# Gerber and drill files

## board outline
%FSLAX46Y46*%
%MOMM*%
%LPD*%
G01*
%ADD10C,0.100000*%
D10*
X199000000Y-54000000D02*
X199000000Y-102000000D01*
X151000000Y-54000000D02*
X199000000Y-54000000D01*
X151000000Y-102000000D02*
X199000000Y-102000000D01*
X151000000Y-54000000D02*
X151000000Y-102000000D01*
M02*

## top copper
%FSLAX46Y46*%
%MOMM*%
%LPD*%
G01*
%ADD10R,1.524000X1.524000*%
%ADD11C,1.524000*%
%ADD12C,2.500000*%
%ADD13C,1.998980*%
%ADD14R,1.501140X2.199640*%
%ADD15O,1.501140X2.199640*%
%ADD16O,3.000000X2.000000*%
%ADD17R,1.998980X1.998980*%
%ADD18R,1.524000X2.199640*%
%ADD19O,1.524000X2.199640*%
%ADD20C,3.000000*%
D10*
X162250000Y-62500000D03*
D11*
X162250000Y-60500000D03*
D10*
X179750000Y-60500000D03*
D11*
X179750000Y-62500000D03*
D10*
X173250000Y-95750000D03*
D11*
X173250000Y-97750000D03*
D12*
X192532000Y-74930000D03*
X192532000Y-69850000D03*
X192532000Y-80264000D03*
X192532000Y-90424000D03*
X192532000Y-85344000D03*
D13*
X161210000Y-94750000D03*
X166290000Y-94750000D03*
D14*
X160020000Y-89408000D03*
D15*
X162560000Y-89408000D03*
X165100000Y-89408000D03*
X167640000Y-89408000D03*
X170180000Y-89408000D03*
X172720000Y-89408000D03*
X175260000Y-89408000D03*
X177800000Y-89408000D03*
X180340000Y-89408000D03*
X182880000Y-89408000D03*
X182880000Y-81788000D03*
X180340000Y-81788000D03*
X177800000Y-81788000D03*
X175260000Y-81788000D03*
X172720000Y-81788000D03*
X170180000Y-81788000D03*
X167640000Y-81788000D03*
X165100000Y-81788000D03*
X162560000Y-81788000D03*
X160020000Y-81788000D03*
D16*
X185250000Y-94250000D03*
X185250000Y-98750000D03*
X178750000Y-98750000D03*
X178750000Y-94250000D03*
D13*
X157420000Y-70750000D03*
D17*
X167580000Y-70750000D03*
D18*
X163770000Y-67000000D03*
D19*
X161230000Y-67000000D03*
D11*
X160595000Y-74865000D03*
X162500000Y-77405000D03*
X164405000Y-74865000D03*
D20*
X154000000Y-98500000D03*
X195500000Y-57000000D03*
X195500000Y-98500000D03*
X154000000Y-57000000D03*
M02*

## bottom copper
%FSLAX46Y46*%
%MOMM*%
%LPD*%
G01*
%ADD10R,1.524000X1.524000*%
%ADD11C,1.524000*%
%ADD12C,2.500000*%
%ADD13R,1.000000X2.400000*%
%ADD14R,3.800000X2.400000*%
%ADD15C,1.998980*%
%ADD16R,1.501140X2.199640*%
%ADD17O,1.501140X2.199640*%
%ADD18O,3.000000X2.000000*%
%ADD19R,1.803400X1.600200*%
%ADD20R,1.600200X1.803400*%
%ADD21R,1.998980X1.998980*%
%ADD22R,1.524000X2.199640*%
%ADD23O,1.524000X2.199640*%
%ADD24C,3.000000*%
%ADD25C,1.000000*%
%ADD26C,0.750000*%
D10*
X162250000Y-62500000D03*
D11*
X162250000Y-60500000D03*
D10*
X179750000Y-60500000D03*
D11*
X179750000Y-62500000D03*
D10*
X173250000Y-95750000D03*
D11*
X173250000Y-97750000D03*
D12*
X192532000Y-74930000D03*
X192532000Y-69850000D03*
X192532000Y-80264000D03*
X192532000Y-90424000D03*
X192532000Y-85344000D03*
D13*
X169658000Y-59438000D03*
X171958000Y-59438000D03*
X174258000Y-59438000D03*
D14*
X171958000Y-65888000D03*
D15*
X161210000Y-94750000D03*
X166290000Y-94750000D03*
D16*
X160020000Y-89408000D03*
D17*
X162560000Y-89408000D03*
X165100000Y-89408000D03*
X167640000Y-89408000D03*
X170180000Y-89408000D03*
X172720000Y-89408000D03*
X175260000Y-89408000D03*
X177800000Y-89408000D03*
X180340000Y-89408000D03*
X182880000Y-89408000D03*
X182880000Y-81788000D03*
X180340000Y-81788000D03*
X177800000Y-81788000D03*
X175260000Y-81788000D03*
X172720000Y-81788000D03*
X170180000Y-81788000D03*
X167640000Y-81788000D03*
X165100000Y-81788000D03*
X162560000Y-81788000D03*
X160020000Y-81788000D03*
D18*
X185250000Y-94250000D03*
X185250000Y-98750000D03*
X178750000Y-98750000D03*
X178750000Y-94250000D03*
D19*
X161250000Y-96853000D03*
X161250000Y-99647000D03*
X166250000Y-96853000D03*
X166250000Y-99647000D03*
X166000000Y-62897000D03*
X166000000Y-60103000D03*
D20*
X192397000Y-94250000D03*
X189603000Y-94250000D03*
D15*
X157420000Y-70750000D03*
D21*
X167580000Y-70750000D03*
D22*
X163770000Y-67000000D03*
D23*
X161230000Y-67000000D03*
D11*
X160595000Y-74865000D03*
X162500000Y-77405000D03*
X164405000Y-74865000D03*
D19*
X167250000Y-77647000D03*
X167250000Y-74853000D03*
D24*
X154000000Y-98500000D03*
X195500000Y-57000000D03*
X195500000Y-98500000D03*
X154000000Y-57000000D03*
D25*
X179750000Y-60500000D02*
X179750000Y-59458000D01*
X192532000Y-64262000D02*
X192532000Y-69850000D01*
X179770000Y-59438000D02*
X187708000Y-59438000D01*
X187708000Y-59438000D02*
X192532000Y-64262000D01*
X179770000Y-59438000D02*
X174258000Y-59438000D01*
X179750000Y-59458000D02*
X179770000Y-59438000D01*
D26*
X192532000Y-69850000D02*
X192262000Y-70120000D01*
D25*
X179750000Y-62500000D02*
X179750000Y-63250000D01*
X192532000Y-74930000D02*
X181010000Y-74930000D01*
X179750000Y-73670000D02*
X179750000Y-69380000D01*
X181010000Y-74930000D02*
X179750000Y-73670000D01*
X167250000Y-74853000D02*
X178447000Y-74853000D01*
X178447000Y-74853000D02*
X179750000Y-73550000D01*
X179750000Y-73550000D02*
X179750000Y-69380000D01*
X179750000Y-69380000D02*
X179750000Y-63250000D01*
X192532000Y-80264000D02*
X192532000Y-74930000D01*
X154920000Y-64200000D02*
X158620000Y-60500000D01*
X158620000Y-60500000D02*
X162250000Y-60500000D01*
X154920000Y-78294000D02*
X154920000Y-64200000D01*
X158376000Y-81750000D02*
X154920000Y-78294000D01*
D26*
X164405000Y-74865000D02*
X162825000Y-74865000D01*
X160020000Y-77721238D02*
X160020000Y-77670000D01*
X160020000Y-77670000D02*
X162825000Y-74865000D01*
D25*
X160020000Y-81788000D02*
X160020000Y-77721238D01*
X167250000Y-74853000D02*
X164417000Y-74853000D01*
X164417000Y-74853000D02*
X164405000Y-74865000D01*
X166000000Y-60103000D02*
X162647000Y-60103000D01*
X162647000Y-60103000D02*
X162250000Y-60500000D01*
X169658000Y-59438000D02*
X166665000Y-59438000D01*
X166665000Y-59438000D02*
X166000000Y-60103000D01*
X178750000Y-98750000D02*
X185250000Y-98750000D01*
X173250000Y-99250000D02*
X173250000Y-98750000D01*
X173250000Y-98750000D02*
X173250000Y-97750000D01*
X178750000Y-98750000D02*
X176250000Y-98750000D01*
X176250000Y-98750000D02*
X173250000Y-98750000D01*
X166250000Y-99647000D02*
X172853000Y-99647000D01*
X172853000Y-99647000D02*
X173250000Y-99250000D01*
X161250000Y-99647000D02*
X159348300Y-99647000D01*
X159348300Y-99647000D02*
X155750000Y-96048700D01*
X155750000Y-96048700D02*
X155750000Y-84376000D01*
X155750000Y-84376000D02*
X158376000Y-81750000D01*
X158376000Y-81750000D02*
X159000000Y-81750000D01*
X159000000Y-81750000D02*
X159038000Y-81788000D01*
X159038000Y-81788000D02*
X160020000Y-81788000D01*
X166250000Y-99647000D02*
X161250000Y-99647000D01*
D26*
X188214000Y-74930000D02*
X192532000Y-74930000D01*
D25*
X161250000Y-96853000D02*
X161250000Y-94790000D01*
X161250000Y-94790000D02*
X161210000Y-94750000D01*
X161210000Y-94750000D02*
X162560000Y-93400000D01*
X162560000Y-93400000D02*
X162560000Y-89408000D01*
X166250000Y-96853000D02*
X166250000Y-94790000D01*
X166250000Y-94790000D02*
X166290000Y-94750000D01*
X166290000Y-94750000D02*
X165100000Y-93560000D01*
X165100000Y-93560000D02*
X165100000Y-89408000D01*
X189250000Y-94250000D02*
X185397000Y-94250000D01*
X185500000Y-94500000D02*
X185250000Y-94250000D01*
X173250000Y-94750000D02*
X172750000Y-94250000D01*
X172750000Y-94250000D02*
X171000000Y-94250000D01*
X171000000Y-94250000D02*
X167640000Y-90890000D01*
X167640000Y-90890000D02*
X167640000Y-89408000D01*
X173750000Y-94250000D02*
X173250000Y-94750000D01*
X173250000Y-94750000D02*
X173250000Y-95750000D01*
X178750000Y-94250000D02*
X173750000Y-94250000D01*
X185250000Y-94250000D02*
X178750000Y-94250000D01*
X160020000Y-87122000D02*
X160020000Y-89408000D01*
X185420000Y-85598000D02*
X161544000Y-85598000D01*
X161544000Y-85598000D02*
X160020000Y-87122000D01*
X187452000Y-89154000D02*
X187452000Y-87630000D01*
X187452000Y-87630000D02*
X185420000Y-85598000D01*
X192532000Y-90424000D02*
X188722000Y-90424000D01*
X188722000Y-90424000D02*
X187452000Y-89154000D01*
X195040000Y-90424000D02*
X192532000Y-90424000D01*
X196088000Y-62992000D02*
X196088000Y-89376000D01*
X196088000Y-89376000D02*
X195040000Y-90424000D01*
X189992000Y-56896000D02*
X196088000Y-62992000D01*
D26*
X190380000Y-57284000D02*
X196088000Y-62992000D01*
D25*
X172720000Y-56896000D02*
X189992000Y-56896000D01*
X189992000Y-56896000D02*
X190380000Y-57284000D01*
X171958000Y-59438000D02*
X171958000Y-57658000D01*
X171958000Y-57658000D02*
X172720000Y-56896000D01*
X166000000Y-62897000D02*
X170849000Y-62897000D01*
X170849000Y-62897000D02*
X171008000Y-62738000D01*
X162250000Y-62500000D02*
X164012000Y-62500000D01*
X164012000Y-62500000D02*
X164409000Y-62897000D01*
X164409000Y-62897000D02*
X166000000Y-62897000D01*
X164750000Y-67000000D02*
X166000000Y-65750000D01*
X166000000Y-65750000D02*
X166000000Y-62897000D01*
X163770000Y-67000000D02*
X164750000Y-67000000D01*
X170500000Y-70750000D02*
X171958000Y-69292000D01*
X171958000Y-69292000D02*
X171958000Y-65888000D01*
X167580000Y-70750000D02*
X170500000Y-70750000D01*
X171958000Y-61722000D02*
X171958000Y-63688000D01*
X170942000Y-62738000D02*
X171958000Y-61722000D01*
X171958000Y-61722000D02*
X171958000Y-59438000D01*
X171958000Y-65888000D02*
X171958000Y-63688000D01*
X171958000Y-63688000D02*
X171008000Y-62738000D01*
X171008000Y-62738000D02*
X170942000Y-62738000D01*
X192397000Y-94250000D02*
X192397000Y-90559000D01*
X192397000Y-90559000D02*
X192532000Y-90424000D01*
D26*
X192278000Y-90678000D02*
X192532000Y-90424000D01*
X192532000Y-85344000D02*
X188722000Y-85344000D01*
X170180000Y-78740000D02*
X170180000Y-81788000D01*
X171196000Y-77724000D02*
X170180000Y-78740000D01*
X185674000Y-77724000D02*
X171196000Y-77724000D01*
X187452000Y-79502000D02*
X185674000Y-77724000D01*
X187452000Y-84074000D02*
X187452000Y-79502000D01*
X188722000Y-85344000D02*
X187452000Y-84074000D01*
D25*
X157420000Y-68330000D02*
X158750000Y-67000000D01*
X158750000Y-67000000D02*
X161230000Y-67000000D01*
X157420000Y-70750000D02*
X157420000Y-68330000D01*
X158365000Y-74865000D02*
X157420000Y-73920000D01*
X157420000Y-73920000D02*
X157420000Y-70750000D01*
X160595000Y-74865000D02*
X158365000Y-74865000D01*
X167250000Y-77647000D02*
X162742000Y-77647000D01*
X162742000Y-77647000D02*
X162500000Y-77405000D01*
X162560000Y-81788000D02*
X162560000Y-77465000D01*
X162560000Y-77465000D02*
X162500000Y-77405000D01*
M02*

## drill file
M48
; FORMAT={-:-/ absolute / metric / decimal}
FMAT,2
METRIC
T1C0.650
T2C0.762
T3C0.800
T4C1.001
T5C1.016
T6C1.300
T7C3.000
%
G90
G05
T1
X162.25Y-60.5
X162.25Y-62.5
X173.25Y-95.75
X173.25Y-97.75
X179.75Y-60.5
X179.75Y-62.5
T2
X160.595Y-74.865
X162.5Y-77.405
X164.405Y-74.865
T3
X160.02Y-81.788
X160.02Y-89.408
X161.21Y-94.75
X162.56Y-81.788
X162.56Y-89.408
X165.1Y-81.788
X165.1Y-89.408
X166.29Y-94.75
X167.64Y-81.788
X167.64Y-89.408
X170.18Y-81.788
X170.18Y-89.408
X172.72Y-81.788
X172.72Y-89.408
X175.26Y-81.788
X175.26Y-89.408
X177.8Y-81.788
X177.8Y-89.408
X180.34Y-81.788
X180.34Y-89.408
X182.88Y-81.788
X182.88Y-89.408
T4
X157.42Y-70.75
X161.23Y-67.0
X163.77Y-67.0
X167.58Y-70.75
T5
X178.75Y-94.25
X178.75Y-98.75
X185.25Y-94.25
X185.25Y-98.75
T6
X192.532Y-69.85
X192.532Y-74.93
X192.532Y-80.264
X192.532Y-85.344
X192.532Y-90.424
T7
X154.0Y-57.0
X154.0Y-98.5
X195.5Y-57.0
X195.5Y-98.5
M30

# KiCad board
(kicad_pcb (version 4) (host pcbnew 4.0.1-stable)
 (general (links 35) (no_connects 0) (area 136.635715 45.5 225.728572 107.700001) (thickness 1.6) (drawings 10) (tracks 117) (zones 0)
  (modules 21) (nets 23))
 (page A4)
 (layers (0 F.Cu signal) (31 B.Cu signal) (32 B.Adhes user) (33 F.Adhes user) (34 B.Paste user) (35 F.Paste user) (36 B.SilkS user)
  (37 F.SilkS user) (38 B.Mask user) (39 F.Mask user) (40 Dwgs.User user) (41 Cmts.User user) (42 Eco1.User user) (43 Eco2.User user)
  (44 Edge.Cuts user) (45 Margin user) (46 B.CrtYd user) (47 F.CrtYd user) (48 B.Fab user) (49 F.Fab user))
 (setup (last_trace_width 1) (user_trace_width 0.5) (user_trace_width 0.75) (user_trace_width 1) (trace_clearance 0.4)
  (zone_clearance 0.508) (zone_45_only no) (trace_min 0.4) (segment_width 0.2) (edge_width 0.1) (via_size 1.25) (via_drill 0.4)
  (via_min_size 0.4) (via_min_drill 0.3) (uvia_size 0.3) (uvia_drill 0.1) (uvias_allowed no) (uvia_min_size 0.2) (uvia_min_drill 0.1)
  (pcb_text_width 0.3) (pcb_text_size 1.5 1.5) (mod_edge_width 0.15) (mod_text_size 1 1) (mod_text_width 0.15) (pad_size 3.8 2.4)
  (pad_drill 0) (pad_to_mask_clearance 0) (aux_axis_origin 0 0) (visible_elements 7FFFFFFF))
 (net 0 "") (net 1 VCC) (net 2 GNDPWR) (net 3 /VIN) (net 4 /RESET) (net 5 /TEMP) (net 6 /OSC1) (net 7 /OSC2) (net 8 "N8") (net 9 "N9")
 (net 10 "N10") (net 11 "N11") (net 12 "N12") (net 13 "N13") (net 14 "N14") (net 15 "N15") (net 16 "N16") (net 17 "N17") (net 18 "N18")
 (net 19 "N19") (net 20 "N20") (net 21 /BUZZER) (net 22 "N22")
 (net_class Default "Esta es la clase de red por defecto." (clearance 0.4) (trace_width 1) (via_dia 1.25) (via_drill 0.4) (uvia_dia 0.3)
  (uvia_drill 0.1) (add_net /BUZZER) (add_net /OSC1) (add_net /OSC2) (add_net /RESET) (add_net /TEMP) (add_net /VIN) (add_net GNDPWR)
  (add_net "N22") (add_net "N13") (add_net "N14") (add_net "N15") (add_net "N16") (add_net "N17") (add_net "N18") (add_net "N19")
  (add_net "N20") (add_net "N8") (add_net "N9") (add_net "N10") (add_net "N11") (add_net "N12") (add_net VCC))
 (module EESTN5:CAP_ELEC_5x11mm (layer F.Cu) (at 162.25 61.5)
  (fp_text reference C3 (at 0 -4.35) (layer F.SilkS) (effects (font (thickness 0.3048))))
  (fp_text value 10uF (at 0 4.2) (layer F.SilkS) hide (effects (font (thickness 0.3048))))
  (pad 1 thru_hole rect (at 0 1) (size 1.524 1.524) (drill 0.65) (layers *.Cu *.Mask F.SilkS) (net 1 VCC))
  (pad 2 thru_hole circle (at 0 -1) (size 1.524 1.524) (drill 0.65) (layers *.Cu *.Mask F.SilkS) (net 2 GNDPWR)))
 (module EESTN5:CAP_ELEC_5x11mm (layer F.Cu) (at 179.75 61.5 180)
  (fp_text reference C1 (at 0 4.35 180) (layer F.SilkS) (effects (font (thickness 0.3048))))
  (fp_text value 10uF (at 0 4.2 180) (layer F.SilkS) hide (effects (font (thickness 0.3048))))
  (pad 1 thru_hole rect (at 0 1 180) (size 1.524 1.524) (drill 0.65) (layers *.Cu *.Mask F.SilkS) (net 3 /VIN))
  (pad 2 thru_hole circle (at 0 -1 180) (size 1.524 1.524) (drill 0.65) (layers *.Cu *.Mask F.SilkS) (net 2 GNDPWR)))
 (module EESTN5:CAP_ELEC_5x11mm (layer F.Cu) (at 173.25 96.75 180)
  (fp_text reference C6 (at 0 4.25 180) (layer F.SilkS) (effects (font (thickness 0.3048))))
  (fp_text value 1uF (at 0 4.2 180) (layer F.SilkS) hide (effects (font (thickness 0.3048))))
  (pad 1 thru_hole rect (at 0 1 180) (size 1.524 1.524) (drill 0.65) (layers *.Cu *.Mask F.SilkS) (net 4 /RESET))
  (pad 2 thru_hole circle (at 0 -1 180) (size 1.524 1.524) (drill 0.65) (layers *.Cu *.Mask F.SilkS) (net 2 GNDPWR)))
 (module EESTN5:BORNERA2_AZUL (layer F.Cu) (at 192.532 72.39 90)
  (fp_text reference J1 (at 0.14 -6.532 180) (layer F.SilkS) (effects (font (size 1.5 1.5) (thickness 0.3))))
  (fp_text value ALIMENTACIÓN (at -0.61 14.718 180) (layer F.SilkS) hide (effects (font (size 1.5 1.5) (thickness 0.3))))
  (pad 1 thru_hole circle (at -2.54 0 90) (size 2.5 2.5) (drill 1.3) (layers *.Cu *.Mask F.SilkS) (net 2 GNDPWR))
  (pad 2 thru_hole circle (at 2.54 0 90) (size 2.5 2.5) (drill 1.3) (layers *.Cu *.Mask F.SilkS) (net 3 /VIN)))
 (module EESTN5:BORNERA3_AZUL (layer F.Cu) (at 192.532 85.344 90)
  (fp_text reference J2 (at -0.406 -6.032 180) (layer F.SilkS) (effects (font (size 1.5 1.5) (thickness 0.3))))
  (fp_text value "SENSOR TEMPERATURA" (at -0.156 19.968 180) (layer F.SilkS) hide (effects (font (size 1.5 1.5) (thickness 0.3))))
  (pad 3 thru_hole circle (at 5.08 0 90) (size 2.5 2.5) (drill 1.3) (layers *.Cu *.Mask F.SilkS) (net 2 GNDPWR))
  (pad 1 thru_hole circle (at -5.08 0 90) (size 2.5 2.5) (drill 1.3) (layers *.Cu *.Mask F.SilkS) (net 1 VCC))
  (pad 2 thru_hole circle (at 0 0 90) (size 2.5 2.5) (drill 1.3) (layers *.Cu *.Mask F.SilkS) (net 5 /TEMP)))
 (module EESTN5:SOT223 (layer B.Cu) (at 171.958 62.738)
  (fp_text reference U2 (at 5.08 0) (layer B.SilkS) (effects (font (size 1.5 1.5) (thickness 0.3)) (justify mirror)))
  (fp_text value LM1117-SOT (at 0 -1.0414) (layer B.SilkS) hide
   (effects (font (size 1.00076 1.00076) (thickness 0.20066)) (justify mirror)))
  (pad 1 smd rect (at -2.3 -3.3) (size 1 2.4) (layers B.Cu B.Paste B.Mask) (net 2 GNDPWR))
  (pad 2 smd rect (at 0 -3.3) (size 1 2.4) (layers B.Cu B.Paste B.Mask) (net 1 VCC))
  (pad 3 smd rect (at 2.3 -3.3) (size 1 2.4) (layers B.Cu B.Paste B.Mask) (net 3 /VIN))
  (pad 4 smd rect (at 0 3.15) (size 3.8 2.4) (layers B.Cu B.Paste B.Mask)))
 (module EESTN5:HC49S (layer F.Cu) (at 163.75 94.75) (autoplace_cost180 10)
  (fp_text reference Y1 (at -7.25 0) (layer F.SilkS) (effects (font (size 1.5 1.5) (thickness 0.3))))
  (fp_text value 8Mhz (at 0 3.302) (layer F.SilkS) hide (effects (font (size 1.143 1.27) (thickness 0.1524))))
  (pad 1 thru_hole circle (at -2.54 0) (size 1.99898 1.99898) (drill 0.8001) (layers *.Cu *.Mask F.SilkS) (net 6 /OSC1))
  (pad 2 thru_hole circle (at 2.54 0) (size 1.99898 1.99898) (drill 0.8001) (layers *.Cu *.Mask F.SilkS) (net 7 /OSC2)))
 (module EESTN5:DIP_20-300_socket (layer F.Cu) (at 171.45 85.598)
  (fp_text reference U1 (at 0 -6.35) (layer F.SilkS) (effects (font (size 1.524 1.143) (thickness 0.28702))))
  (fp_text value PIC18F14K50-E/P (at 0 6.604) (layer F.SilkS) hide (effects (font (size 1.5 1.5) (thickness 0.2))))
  (pad 1 thru_hole rect (at -11.43 3.81) (size 1.50114 2.19964) (drill 0.8001) (layers *.Cu *.Mask F.SilkS) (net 1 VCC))
  (pad 2 thru_hole oval (at -8.89 3.81) (size 1.50114 2.19964) (drill 0.8001) (layers *.Cu *.Mask F.SilkS) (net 6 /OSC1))
  (pad 3 thru_hole oval (at -6.35 3.81) (size 1.50114 2.19964) (drill 0.8001) (layers *.Cu *.Mask F.SilkS) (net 7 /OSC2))
  (pad 4 thru_hole oval (at -3.81 3.81) (size 1.50114 2.19964) (drill 0.8001) (layers *.Cu *.Mask F.SilkS) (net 4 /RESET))
  (pad 5 thru_hole oval (at -1.27 3.81) (size 1.50114 2.19964) (drill 0.8001) (layers *.Cu *.Mask F.SilkS) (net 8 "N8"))
  (pad 6 thru_hole oval (at 1.27 3.81) (size 1.50114 2.19964) (drill 0.8001) (layers *.Cu *.Mask F.SilkS) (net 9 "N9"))
  (pad 7 thru_hole oval (at 3.81 3.81) (size 1.50114 2.19964) (drill 0.8001) (layers *.Cu *.Mask F.SilkS) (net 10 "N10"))
  (pad 8 thru_hole oval (at 6.35 3.81) (size 1.50114 2.19964) (drill 0.8001) (layers *.Cu *.Mask F.SilkS) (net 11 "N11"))
  (pad 9 thru_hole oval (at 8.89 3.81) (size 1.50114 2.19964) (drill 0.8001) (layers *.Cu *.Mask F.SilkS) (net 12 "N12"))
  (pad 10 thru_hole oval (at 11.43 3.81) (size 1.50114 2.19964) (drill 0.8001) (layers *.Cu *.Mask F.SilkS) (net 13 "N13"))
  (pad 11 thru_hole oval (at 11.43 -3.81) (size 1.50114 2.19964) (drill 0.8001) (layers *.Cu *.Mask F.SilkS) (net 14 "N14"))
  (pad 12 thru_hole oval (at 8.89 -3.81) (size 1.50114 2.19964) (drill 0.8001) (layers *.Cu *.Mask F.SilkS) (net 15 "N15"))
  (pad 13 thru_hole oval (at 6.35 -3.81) (size 1.50114 2.19964) (drill 0.8001) (layers *.Cu *.Mask F.SilkS) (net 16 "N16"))
  (pad 14 thru_hole oval (at 3.81 -3.81) (size 1.50114 2.19964) (drill 0.8001) (layers *.Cu *.Mask F.SilkS) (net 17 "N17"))
  (pad 15 thru_hole oval (at 1.27 -3.81) (size 1.50114 2.19964) (drill 0.8001) (layers *.Cu *.Mask F.SilkS) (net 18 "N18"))
  (pad 16 thru_hole oval (at -1.27 -3.81) (size 1.50114 2.19964) (drill 0.8001) (layers *.Cu *.Mask F.SilkS) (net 5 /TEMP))
  (pad 17 thru_hole oval (at -3.81 -3.81) (size 1.50114 2.19964) (drill 0.8001) (layers *.Cu *.Mask F.SilkS) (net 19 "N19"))
  (pad 18 thru_hole oval (at -6.35 -3.81) (size 1.50114 2.19964) (drill 0.8001) (layers *.Cu *.Mask F.SilkS) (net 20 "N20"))
  (pad 19 thru_hole oval (at -8.89 -3.81) (size 1.50114 2.19964) (drill 0.8001) (layers *.Cu *.Mask F.SilkS) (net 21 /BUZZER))
  (pad 20 thru_hole oval (at -11.43 -3.81) (size 1.50114 2.19964) (drill 0.8001) (layers *.Cu *.Mask F.SilkS) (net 2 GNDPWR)))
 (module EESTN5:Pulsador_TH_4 (layer F.Cu) (at 185.25 94.25 270)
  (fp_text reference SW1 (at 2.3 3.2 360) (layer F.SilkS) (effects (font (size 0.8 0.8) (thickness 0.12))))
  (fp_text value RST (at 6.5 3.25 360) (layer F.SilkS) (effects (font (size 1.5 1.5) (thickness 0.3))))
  (pad 3 thru_hole oval (at 0 0 270) (size 2 3) (drill 1.016) (layers *.Cu *.Mask F.SilkS) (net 4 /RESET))
  (pad 1 thru_hole oval (at 4.5 0 270) (size 2 3) (drill 1.016) (layers *.Cu *.Mask F.SilkS) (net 2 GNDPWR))
  (pad 2 thru_hole oval (at 4.5 6.5 270) (size 2 3) (drill 1.016) (layers *.Cu *.Mask F.SilkS) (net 2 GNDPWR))
  (pad 4 thru_hole oval (at 0 6.5 270) (size 2 3) (drill 1.016) (layers *.Cu *.Mask F.SilkS) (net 4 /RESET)))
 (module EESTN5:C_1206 (layer B.Cu) (at 161.25 98.25 90)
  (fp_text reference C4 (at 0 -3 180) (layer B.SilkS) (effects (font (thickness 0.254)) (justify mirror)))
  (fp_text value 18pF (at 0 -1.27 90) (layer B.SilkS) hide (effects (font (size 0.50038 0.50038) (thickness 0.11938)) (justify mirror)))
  (pad 1 smd rect (at 1.397 0 90) (size 1.6002 1.8034) (layers B.Cu B.Paste B.Mask) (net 6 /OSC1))
  (pad 2 smd rect (at -1.397 0 90) (size 1.6002 1.8034) (layers B.Cu B.Paste B.Mask) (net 2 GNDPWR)))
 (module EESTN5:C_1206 (layer B.Cu) (at 166.25 98.25 90)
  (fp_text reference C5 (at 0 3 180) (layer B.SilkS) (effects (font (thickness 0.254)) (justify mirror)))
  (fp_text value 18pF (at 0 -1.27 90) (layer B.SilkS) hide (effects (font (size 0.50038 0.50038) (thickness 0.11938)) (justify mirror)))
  (pad 1 smd rect (at 1.397 0 90) (size 1.6002 1.8034) (layers B.Cu B.Paste B.Mask) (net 7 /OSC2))
  (pad 2 smd rect (at -1.397 0 90) (size 1.6002 1.8034) (layers B.Cu B.Paste B.Mask) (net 2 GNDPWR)))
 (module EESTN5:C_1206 (layer B.Cu) (at 166 61.5 270)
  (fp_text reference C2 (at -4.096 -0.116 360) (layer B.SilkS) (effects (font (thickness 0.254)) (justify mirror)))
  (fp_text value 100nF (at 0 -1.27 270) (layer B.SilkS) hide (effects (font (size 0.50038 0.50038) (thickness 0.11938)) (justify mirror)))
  (pad 1 smd rect (at 1.397 0 270) (size 1.6002 1.8034) (layers B.Cu B.Paste B.Mask) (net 1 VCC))
  (pad 2 smd rect (at -1.397 0 270) (size 1.6002 1.8034) (layers B.Cu B.Paste B.Mask) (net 2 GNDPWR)))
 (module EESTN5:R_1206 (layer B.Cu) (at 191 94.25)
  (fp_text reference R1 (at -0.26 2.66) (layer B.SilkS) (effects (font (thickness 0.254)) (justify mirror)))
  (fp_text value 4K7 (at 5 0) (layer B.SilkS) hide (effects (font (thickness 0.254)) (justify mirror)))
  (pad 1 smd rect (at 1.397 0) (size 1.6002 1.8034) (layers B.Cu B.Paste B.Mask) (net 1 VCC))
  (pad 2 smd rect (at -1.397 0) (size 1.6002 1.8034) (layers B.Cu B.Paste B.Mask) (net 4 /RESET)))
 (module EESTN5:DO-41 (layer F.Cu) (at 162.5 70.75)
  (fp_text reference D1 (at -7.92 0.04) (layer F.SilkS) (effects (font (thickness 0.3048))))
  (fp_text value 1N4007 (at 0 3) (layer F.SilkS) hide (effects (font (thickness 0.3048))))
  (pad 1 thru_hole circle (at -5.08 0) (size 1.99898 1.99898) (drill 1.00076) (layers *.Cu *.Mask F.SilkS) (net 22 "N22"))
  (pad 2 thru_hole rect (at 5.08 0) (size 1.99898 1.99898) (drill 1.00076) (layers *.Cu *.Mask F.SilkS) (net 1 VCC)))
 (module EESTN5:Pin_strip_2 (layer F.Cu) (at 162.5 67 180)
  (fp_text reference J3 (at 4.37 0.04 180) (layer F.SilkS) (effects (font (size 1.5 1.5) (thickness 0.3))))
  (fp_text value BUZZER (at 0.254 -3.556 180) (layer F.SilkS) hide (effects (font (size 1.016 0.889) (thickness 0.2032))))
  (pad 1 thru_hole rect (at -1.27 0 180) (size 1.524 2.19964) (drill 1.00076) (layers *.Cu *.Mask F.SilkS) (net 1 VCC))
  (pad 2 thru_hole oval (at 1.27 0 180) (size 1.524 2.19964) (drill 1.00076) (layers *.Cu *.Mask F.SilkS) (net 22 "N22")))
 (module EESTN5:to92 (layer F.Cu) (at 162.5 75.5 180)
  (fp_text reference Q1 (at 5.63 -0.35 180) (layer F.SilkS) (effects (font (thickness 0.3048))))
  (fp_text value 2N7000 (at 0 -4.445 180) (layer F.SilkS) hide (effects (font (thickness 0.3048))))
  (pad 3 thru_hole circle (at 1.905 0.635 180) (size 1.524 1.524) (drill 0.762) (layers *.Cu *.Mask F.SilkS) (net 22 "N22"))
  (pad 2 thru_hole circle (at 0 -1.905 180) (size 1.524 1.524) (drill 0.762) (layers *.Cu *.Mask F.SilkS) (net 21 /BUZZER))
  (pad 1 thru_hole circle (at -1.905 0.635 180) (size 1.524 1.524) (drill 0.762) (layers *.Cu *.Mask F.SilkS) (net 2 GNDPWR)))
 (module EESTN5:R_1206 (layer B.Cu) (at 167.25 76.25 270)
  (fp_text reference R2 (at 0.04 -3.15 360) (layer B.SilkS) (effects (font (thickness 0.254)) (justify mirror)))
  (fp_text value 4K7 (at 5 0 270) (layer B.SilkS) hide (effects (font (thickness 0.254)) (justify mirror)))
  (pad 1 smd rect (at 1.397 0 270) (size 1.6002 1.8034) (layers B.Cu B.Paste B.Mask) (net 21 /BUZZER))
  (pad 2 smd rect (at -1.397 0 270) (size 1.6002 1.8034) (layers B.Cu B.Paste B.Mask) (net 2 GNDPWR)))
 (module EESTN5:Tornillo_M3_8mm (layer F.Cu) (at 154 98.5)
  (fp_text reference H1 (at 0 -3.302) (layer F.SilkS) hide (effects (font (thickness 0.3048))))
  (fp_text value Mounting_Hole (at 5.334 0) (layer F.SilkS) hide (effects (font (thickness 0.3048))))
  (pad 1 thru_hole circle (at 0 0) (size 3 3) (drill 3) (layers *.Cu F.SilkS)))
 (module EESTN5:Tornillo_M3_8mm (layer F.Cu) (at 195.5 57)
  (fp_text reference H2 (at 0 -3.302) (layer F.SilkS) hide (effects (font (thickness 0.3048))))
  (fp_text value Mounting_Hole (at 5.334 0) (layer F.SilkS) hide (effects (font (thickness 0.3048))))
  (pad 1 thru_hole circle (at 0 0) (size 3 3) (drill 3) (layers *.Cu F.SilkS)))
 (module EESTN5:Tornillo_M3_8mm (layer F.Cu) (at 195.5 98.5)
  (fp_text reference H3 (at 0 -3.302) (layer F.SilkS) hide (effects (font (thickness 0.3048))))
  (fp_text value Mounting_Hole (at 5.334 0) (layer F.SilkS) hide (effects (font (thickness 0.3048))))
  (pad 1 thru_hole circle (at 0 0) (size 3 3) (drill 3) (layers *.Cu F.SilkS)))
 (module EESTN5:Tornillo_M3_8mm (layer F.Cu) (at 154 57)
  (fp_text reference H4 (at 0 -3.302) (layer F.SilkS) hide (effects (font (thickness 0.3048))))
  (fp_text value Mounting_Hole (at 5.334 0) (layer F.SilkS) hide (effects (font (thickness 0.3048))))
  (pad 1 thru_hole circle (at 0 0) (size 3 3) (drill 3) (layers *.Cu F.SilkS)))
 (gr_line (start 199 54) (end 199 102) (angle 90) (layer Edge.Cuts) (width 0.1))
 (gr_line (start 151 54) (end 199 54) (angle 90) (layer Edge.Cuts) (width 0.1))
 (gr_line (start 151 102) (end 199 102) (angle 90) (layer Edge.Cuts) (width 0.1))
 (gr_line (start 151 54) (end 151 102) (angle 90) (layer Edge.Cuts) (width 0.1))
 (segment (start 179.75 60.5) (end 179.75 59.458) (width 1) (layer B.Cu) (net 3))
 (segment (start 192.532 64.262) (end 192.532 69.85) (width 1) (layer B.Cu) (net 3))
 (segment (start 179.77 59.438) (end 187.708 59.438) (width 1) (layer B.Cu) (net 3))
 (segment (start 187.708 59.438) (end 192.532 64.262) (width 1) (layer B.Cu) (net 3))
 (segment (start 179.77 59.438) (end 174.258 59.438) (width 1) (layer B.Cu) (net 3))
 (segment (start 179.75 59.458) (end 179.77 59.438) (width 1) (layer B.Cu) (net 3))
 (segment (start 192.532 69.85) (end 192.262 70.12) (width 0.75) (layer B.Cu) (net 3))
 (segment (start 179.75 62.5) (end 179.75 63.25) (width 1) (layer B.Cu) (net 2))
 (segment (start 192.532 74.93) (end 181.01 74.93) (width 1) (layer B.Cu) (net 2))
 (segment (start 179.75 73.67) (end 179.75 69.38) (width 1) (layer B.Cu) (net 2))
 (segment (start 181.01 74.93) (end 179.75 73.67) (width 1) (layer B.Cu) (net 2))
 (segment (start 167.25 74.853) (end 178.447 74.853) (width 1) (layer B.Cu) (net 2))
 (segment (start 178.447 74.853) (end 179.75 73.55) (width 1) (layer B.Cu) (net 2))
 (segment (start 179.75 73.55) (end 179.75 69.38) (width 1) (layer B.Cu) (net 2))
 (segment (start 179.75 69.38) (end 179.75 63.25) (width 1) (layer B.Cu) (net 2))
 (segment (start 192.532 80.264) (end 192.532 74.93) (width 1) (layer B.Cu) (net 2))
 (segment (start 154.92 64.2) (end 158.62 60.5) (width 1) (layer B.Cu) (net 2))
 (segment (start 158.62 60.5) (end 162.25 60.5) (width 1) (layer B.Cu) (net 2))
 (segment (start 154.92 78.294) (end 154.92 64.2) (width 1) (layer B.Cu) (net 2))
 (segment (start 158.376 81.75) (end 154.92 78.294) (width 1) (layer B.Cu) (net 2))
 (segment (start 164.405 74.865) (end 162.825 74.865) (width 0.75) (layer B.Cu) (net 2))
 (segment (start 160.02 77.721238) (end 160.02 77.67) (width 0.75) (layer B.Cu) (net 2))
 (segment (start 160.02 77.67) (end 162.825 74.865) (width 0.75) (layer B.Cu) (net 2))
 (segment (start 160.02 81.788) (end 160.02 77.721238) (width 1) (layer B.Cu) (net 2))
 (segment (start 167.25 74.853) (end 164.417 74.853) (width 1) (layer B.Cu) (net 2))
 (segment (start 164.417 74.853) (end 164.405 74.865) (width 1) (layer B.Cu) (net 2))
 (segment (start 166 60.103) (end 162.647 60.103) (width 1) (layer B.Cu) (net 2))
 (segment (start 162.647 60.103) (end 162.25 60.5) (width 1) (layer B.Cu) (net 2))
 (segment (start 169.658 59.438) (end 166.665 59.438) (width 1) (layer B.Cu) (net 2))
 (segment (start 166.665 59.438) (end 166 60.103) (width 1) (layer B.Cu) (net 2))
 (segment (start 178.75 98.75) (end 185.25 98.75) (width 1) (layer B.Cu) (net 2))
 (segment (start 173.25 99.25) (end 173.25 98.75) (width 1) (layer B.Cu) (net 2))
 (segment (start 173.25 98.75) (end 173.25 97.75) (width 1) (layer B.Cu) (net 2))
 (segment (start 178.75 98.75) (end 176.25 98.75) (width 1) (layer B.Cu) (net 2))
 (segment (start 176.25 98.75) (end 173.25 98.75) (width 1) (layer B.Cu) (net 2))
 (segment (start 166.25 99.647) (end 172.853 99.647) (width 1) (layer B.Cu) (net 2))
 (segment (start 172.853 99.647) (end 173.25 99.25) (width 1) (layer B.Cu) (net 2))
 (segment (start 161.25 99.647) (end 159.3483 99.647) (width 1) (layer B.Cu) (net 2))
 (segment (start 159.3483 99.647) (end 155.75 96.0487) (width 1) (layer B.Cu) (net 2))
 (segment (start 155.75 96.0487) (end 155.75 84.376) (width 1) (layer B.Cu) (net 2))
 (segment (start 155.75 84.376) (end 158.376 81.75) (width 1) (layer B.Cu) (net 2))
 (segment (start 158.376 81.75) (end 159 81.75) (width 1) (layer B.Cu) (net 2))
 (segment (start 159 81.75) (end 159.038 81.788) (width 1) (layer B.Cu) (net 2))
 (segment (start 159.038 81.788) (end 160.02 81.788) (width 1) (layer B.Cu) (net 2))
 (segment (start 166.25 99.647) (end 161.25 99.647) (width 1) (layer B.Cu) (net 2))
 (segment (start 188.214 74.93) (end 192.532 74.93) (width 0.75) (layer B.Cu) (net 2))
 (segment (start 161.25 96.853) (end 161.25 94.79) (width 1) (layer B.Cu) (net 6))
 (segment (start 161.25 94.79) (end 161.21 94.75) (width 1) (layer B.Cu) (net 6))
 (segment (start 161.21 94.75) (end 162.56 93.4) (width 1) (layer B.Cu) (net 6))
 (segment (start 162.56 93.4) (end 162.56 89.408) (width 1) (layer B.Cu) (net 6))
 (segment (start 166.25 96.853) (end 166.25 94.79) (width 1) (layer B.Cu) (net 7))
 (segment (start 166.25 94.79) (end 166.29 94.75) (width 1) (layer B.Cu) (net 7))
 (segment (start 166.29 94.75) (end 165.1 93.56) (width 1) (layer B.Cu) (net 7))
 (segment (start 165.1 93.56) (end 165.1 89.408) (width 1) (layer B.Cu) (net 7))
 (segment (start 189.25 94.25) (end 185.397 94.25) (width 1) (layer B.Cu) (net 4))
 (segment (start 185.5 94.5) (end 185.25 94.25) (width 1) (layer B.Cu) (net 4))
 (segment (start 173.25 94.75) (end 172.75 94.25) (width 1) (layer B.Cu) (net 4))
 (segment (start 172.75 94.25) (end 171 94.25) (width 1) (layer B.Cu) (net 4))
 (segment (start 171 94.25) (end 167.64 90.89) (width 1) (layer B.Cu) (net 4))
 (segment (start 167.64 90.89) (end 167.64 89.408) (width 1) (layer B.Cu) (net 4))
 (segment (start 173.75 94.25) (end 173.25 94.75) (width 1) (layer B.Cu) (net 4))
 (segment (start 173.25 94.75) (end 173.25 95.75) (width 1) (layer B.Cu) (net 4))
 (segment (start 178.75 94.25) (end 173.75 94.25) (width 1) (layer B.Cu) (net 4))
 (segment (start 185.25 94.25) (end 178.75 94.25) (width 1) (layer B.Cu) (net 4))
 (segment (start 160.02 87.122) (end 160.02 89.408) (width 1) (layer B.Cu) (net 1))
 (segment (start 185.42 85.598) (end 161.544 85.598) (width 1) (layer B.Cu) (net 1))
 (segment (start 161.544 85.598) (end 160.02 87.122) (width 1) (layer B.Cu) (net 1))
 (segment (start 187.452 89.154) (end 187.452 87.63) (width 1) (layer B.Cu) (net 1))
 (segment (start 187.452 87.63) (end 185.42 85.598) (width 1) (layer B.Cu) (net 1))
 (segment (start 192.532 90.424) (end 188.722 90.424) (width 1) (layer B.Cu) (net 1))
 (segment (start 188.722 90.424) (end 187.452 89.154) (width 1) (layer B.Cu) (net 1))
 (segment (start 195.04 90.424) (end 192.532 90.424) (width 1) (layer B.Cu) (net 1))
 (segment (start 196.088 62.992) (end 196.088 89.376) (width 1) (layer B.Cu) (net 1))
 (segment (start 196.088 89.376) (end 195.04 90.424) (width 1) (layer B.Cu) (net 1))
 (segment (start 189.992 56.896) (end 196.088 62.992) (width 1) (layer B.Cu) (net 1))
 (segment (start 190.38 57.284) (end 196.088 62.992) (width 0.75) (layer B.Cu) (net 1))
 (segment (start 172.72 56.896) (end 189.992 56.896) (width 1) (layer B.Cu) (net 1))
 (segment (start 189.992 56.896) (end 190.38 57.284) (width 1) (layer B.Cu) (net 1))
 (segment (start 171.958 59.438) (end 171.958 57.658) (width 1) (layer B.Cu) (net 1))
 (segment (start 171.958 57.658) (end 172.72 56.896) (width 1) (layer B.Cu) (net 1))
 (segment (start 166 62.897) (end 170.849 62.897) (width 1) (layer B.Cu) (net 1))
 (segment (start 170.849 62.897) (end 171.008 62.738) (width 1) (layer B.Cu) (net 1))
 (segment (start 162.25 62.5) (end 164.012 62.5) (width 1) (layer B.Cu) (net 1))
 (segment (start 164.012 62.5) (end 164.409 62.897) (width 1) (layer B.Cu) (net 1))
 (segment (start 164.409 62.897) (end 166 62.897) (width 1) (layer B.Cu) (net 1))
 (segment (start 164.75 67) (end 166 65.75) (width 1) (layer B.Cu) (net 1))
 (segment (start 166 65.75) (end 166 62.897) (width 1) (layer B.Cu) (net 1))
 (segment (start 163.77 67) (end 164.75 67) (width 1) (layer B.Cu) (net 1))
 (segment (start 170.5 70.75) (end 171.958 69.292) (width 1) (layer B.Cu) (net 1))
 (segment (start 171.958 69.292) (end 171.958 65.888) (width 1) (layer B.Cu) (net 1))
 (segment (start 167.58 70.75) (end 170.5 70.75) (width 1) (layer B.Cu) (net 1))
 (segment (start 171.958 61.722) (end 171.958 63.688) (width 1) (layer B.Cu) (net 1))
 (segment (start 170.942 62.738) (end 171.958 61.722) (width 1) (layer B.Cu) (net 1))
 (segment (start 171.958 61.722) (end 171.958 59.438) (width 1) (layer B.Cu) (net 1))
 (segment (start 171.958 65.888) (end 171.958 63.688) (width 1) (layer B.Cu) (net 1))
 (segment (start 171.958 63.688) (end 171.008 62.738) (width 1) (layer B.Cu) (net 1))
 (segment (start 171.008 62.738) (end 170.942 62.738) (width 1) (layer B.Cu) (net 1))
 (segment (start 192.397 94.25) (end 192.397 90.559) (width 1) (layer B.Cu) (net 1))
 (segment (start 192.397 90.559) (end 192.532 90.424) (width 1) (layer B.Cu) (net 1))
 (segment (start 192.278 90.678) (end 192.532 90.424) (width 0.75) (layer B.Cu) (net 1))
 (segment (start 192.532 85.344) (end 188.722 85.344) (width 0.75) (layer B.Cu) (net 5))
 (segment (start 170.18 78.74) (end 170.18 81.788) (width 0.75) (layer B.Cu) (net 5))
 (segment (start 171.196 77.724) (end 170.18 78.74) (width 0.75) (layer B.Cu) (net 5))
 (segment (start 185.674 77.724) (end 171.196 77.724) (width 0.75) (layer B.Cu) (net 5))
 (segment (start 187.452 79.502) (end 185.674 77.724) (width 0.75) (layer B.Cu) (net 5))
 (segment (start 187.452 84.074) (end 187.452 79.502) (width 0.75) (layer B.Cu) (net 5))
 (segment (start 188.722 85.344) (end 187.452 84.074) (width 0.75) (layer B.Cu) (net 5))
 (segment (start 157.42 68.33) (end 158.75 67) (width 1) (layer B.Cu) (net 22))
 (segment (start 158.75 67) (end 161.23 67) (width 1) (layer B.Cu) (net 22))
 (segment (start 157.42 70.75) (end 157.42 68.33) (width 1) (layer B.Cu) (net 22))
 (segment (start 158.365 74.865) (end 157.42 73.92) (width 1) (layer B.Cu) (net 22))
 (segment (start 157.42 73.92) (end 157.42 70.75) (width 1) (layer B.Cu) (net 22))
 (segment (start 160.595 74.865) (end 158.365 74.865) (width 1) (layer B.Cu) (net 22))
 (segment (start 167.25 77.647) (end 162.742 77.647) (width 1) (layer B.Cu) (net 21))
 (segment (start 162.742 77.647) (end 162.5 77.405) (width 1) (layer B.Cu) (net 21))
 (segment (start 162.56 81.788) (end 162.56 77.465) (width 1) (layer B.Cu) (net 21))
 (segment (start 162.56 77.465) (end 162.5 77.405) (width 1) (layer B.Cu) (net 21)))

